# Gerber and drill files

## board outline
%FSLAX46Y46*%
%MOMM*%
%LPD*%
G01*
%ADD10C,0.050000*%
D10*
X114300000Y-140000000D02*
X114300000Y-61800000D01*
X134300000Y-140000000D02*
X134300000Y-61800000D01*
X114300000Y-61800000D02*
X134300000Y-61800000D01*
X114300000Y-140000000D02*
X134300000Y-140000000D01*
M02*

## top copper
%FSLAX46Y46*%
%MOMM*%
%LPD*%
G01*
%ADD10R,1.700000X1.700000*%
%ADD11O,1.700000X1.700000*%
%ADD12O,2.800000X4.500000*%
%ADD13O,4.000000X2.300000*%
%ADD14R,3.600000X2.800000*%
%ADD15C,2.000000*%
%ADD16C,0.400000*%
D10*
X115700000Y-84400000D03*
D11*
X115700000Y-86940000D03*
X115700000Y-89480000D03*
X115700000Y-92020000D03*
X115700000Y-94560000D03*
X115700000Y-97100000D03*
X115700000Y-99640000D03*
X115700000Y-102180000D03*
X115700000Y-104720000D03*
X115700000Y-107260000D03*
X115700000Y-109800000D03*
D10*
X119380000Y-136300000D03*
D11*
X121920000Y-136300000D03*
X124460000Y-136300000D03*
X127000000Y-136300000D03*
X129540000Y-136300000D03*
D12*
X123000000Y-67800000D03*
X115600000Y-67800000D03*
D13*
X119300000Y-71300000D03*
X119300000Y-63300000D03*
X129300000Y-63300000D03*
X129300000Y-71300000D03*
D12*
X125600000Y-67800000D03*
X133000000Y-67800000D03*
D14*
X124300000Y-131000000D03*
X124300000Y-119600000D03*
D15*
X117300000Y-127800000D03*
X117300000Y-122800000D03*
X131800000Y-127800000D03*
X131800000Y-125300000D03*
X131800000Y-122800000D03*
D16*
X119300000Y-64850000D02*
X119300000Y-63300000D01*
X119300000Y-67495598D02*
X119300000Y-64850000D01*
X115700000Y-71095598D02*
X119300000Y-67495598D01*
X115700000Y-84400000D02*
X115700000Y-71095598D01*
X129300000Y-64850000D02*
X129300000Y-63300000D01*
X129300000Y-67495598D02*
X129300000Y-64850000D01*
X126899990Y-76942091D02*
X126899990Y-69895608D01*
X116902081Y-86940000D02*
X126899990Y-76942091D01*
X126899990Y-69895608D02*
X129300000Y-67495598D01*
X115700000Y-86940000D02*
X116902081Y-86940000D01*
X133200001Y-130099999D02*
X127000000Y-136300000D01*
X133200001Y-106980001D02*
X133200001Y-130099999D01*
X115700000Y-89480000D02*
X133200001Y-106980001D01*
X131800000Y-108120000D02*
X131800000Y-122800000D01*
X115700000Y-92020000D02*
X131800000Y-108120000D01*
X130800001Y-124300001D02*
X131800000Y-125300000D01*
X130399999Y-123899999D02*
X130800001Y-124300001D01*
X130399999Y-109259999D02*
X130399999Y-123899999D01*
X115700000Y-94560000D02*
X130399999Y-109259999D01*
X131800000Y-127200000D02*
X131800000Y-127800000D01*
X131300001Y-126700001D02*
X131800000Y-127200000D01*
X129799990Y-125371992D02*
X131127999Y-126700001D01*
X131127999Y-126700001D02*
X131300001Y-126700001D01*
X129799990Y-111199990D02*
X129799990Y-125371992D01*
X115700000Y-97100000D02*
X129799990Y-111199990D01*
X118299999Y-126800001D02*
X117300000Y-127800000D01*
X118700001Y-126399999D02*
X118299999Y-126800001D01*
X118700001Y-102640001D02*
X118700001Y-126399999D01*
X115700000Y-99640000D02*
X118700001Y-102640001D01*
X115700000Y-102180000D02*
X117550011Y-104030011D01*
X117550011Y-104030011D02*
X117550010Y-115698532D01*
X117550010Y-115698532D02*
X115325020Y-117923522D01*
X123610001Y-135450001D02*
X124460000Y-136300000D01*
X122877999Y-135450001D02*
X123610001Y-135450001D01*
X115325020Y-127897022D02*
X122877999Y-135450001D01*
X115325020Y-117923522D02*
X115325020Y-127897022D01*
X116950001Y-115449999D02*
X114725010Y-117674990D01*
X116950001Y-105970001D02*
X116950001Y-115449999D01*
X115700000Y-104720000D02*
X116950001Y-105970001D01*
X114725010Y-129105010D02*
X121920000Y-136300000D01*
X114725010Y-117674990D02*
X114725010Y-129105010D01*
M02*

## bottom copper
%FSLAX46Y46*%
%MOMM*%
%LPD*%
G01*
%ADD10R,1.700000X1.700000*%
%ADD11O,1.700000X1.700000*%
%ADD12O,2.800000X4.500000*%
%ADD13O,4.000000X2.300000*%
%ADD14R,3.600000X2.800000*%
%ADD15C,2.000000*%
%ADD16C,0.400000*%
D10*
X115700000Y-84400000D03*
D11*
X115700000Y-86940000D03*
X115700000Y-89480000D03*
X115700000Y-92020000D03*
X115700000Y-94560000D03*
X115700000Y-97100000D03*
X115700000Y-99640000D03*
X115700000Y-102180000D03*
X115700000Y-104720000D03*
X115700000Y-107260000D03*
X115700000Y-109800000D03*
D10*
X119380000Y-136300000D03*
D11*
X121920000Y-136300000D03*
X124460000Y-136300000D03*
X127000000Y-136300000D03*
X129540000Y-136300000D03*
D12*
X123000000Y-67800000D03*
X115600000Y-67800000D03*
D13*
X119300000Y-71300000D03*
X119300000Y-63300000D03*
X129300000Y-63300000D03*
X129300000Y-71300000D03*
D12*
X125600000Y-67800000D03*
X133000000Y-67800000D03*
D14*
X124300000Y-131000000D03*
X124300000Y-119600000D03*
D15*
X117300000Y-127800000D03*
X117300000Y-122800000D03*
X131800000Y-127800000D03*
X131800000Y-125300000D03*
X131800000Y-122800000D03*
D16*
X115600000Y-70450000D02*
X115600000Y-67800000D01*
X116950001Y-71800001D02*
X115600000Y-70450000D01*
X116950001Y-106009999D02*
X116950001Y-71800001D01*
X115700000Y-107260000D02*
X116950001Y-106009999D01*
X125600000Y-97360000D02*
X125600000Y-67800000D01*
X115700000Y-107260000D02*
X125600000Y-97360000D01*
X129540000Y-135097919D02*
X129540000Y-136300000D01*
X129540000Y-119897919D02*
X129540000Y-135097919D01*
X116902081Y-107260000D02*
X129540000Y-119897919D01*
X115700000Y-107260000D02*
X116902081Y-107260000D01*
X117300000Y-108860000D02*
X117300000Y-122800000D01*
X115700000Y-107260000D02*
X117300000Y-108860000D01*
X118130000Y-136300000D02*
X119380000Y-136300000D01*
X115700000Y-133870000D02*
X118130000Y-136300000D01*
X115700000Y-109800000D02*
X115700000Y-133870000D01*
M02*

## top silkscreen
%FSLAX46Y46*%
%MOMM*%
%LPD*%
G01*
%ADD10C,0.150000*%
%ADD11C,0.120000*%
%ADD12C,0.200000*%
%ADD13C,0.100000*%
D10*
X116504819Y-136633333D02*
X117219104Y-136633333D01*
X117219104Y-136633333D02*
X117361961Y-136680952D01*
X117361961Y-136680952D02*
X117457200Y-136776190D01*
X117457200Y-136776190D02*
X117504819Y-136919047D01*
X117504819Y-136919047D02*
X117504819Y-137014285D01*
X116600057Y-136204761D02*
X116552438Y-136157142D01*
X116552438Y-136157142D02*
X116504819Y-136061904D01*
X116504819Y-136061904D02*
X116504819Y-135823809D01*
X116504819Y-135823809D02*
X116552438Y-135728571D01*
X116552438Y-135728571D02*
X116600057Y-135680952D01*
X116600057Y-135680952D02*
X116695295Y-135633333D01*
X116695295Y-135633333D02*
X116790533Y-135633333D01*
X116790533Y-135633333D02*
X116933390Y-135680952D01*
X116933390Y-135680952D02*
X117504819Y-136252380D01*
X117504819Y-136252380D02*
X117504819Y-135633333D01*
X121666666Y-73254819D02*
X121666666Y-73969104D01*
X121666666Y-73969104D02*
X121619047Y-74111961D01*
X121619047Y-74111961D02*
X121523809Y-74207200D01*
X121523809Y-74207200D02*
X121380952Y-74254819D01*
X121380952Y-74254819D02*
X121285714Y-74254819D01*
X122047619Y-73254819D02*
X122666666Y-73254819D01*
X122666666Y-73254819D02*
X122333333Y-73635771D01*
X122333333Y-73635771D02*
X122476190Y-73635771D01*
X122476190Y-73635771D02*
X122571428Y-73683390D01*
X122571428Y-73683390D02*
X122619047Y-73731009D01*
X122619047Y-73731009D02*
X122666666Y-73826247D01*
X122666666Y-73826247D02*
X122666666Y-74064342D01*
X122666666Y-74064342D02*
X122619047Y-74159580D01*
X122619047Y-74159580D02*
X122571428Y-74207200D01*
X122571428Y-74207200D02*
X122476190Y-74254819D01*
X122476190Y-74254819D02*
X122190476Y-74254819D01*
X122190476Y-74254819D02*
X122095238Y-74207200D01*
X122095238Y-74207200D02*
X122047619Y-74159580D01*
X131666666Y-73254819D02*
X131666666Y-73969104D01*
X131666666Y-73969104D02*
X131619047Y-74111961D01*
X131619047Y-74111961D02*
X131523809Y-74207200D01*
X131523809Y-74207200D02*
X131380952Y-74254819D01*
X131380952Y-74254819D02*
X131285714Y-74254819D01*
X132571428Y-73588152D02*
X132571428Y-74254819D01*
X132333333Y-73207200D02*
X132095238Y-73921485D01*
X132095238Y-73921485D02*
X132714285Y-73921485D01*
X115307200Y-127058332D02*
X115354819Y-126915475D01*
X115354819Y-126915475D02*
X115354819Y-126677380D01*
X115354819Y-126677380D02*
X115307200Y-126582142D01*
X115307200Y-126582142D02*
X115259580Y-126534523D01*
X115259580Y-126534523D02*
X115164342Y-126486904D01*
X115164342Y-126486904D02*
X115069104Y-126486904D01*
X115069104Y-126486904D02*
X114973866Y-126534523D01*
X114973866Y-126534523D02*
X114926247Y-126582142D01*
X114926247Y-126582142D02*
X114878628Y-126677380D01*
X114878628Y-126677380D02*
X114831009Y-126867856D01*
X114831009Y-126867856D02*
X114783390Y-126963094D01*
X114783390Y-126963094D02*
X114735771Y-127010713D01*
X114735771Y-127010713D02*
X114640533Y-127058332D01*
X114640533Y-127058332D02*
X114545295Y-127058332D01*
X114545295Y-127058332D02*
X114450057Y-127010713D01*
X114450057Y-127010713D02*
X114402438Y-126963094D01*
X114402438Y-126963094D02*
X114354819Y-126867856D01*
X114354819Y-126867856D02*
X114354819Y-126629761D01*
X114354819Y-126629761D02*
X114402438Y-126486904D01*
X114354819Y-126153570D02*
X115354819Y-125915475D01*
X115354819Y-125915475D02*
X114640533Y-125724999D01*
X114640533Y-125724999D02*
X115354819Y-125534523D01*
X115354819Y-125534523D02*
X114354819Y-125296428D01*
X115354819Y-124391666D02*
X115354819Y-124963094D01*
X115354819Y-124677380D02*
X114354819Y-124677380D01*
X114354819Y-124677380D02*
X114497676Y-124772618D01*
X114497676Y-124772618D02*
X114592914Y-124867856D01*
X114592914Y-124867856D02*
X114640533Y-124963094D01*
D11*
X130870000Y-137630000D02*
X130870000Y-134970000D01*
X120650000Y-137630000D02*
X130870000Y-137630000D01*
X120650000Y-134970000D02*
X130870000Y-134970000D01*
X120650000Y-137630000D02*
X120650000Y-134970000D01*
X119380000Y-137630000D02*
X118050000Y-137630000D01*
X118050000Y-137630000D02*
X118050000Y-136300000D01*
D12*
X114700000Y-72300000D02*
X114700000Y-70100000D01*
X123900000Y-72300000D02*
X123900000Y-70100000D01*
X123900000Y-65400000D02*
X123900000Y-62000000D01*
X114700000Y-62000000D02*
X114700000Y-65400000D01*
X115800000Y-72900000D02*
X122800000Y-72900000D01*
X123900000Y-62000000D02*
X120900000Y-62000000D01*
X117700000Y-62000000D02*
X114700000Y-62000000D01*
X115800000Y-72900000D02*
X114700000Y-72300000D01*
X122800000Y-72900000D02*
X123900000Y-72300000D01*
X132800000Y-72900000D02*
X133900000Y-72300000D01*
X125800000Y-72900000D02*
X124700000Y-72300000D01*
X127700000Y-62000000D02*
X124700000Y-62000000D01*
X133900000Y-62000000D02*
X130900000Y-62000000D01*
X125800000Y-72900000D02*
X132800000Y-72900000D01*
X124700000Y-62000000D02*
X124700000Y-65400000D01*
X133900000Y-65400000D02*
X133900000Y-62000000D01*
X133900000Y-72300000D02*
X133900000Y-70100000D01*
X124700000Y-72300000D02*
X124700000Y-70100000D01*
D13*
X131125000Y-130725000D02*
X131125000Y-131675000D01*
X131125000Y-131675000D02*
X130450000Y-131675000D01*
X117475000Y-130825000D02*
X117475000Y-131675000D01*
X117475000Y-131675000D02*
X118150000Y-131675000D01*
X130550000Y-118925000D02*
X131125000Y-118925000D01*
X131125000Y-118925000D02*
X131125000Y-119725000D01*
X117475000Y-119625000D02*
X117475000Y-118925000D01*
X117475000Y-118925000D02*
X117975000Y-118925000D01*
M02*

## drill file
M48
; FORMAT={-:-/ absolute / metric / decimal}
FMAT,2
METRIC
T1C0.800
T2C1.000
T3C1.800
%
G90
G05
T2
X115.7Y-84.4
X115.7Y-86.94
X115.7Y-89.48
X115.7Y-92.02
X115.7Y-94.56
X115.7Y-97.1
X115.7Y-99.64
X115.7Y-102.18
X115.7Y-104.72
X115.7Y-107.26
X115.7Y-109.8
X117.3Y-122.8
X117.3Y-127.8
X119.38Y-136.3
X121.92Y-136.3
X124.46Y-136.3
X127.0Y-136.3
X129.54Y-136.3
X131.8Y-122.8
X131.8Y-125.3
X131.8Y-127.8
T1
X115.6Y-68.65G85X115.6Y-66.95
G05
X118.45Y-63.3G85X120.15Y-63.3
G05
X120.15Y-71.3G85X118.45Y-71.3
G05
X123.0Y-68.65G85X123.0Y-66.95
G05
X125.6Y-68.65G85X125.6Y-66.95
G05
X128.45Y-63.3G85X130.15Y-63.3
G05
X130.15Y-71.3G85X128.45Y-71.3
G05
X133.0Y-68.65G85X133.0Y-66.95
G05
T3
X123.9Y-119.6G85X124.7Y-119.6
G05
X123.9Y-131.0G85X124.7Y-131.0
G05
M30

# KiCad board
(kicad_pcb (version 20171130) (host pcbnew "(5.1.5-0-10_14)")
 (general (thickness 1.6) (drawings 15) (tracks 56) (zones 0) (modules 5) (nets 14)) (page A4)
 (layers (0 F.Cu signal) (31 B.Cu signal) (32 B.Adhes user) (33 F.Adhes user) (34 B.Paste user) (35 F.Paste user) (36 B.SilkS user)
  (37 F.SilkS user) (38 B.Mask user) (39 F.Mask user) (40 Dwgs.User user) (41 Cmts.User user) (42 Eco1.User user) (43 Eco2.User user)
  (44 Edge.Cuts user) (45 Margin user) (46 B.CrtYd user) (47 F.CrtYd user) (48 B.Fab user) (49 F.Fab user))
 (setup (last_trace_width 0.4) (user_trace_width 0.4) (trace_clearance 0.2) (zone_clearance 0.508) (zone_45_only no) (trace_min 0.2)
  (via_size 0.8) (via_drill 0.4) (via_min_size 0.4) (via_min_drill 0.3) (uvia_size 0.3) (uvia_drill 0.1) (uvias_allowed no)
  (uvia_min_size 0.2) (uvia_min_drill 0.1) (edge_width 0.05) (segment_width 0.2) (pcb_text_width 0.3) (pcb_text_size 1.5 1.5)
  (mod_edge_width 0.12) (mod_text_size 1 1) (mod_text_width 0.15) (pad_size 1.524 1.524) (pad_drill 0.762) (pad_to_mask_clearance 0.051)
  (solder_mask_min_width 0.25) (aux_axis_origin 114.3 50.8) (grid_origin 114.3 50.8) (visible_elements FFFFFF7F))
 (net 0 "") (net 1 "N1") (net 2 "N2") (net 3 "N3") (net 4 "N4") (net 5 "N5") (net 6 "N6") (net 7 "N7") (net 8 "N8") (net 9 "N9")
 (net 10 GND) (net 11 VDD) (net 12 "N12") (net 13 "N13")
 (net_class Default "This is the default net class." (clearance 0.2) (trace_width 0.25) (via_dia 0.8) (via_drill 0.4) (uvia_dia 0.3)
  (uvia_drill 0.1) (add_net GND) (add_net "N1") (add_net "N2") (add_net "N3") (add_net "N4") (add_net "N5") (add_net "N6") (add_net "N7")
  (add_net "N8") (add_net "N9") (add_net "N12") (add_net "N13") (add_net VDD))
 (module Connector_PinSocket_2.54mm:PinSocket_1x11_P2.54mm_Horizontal (layer B.Cu) (at 115.7 84.4 180)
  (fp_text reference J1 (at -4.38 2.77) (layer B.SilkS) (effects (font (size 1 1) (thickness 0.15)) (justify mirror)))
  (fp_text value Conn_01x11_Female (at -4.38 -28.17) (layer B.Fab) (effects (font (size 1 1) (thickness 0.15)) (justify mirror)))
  (pad 1 thru_hole rect (at 0 0 180) (size 1.7 1.7) (drill 1) (layers *.Cu *.Mask) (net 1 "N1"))
  (pad 2 thru_hole oval (at 0 -2.54 180) (size 1.7 1.7) (drill 1) (layers *.Cu *.Mask) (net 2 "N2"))
  (pad 3 thru_hole oval (at 0 -5.08 180) (size 1.7 1.7) (drill 1) (layers *.Cu *.Mask) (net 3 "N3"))
  (pad 4 thru_hole oval (at 0 -7.62 180) (size 1.7 1.7) (drill 1) (layers *.Cu *.Mask) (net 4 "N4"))
  (pad 5 thru_hole oval (at 0 -10.16 180) (size 1.7 1.7) (drill 1) (layers *.Cu *.Mask) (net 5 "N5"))
  (pad 6 thru_hole oval (at 0 -12.7 180) (size 1.7 1.7) (drill 1) (layers *.Cu *.Mask) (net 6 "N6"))
  (pad 7 thru_hole oval (at 0 -15.24 180) (size 1.7 1.7) (drill 1) (layers *.Cu *.Mask) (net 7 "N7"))
  (pad 8 thru_hole oval (at 0 -17.78 180) (size 1.7 1.7) (drill 1) (layers *.Cu *.Mask) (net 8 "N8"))
  (pad 9 thru_hole oval (at 0 -20.32 180) (size 1.7 1.7) (drill 1) (layers *.Cu *.Mask) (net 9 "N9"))
  (pad 10 thru_hole oval (at 0 -22.86 180) (size 1.7 1.7) (drill 1) (layers *.Cu *.Mask) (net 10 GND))
  (pad 11 thru_hole oval (at 0 -25.4 180) (size 1.7 1.7) (drill 1) (layers *.Cu *.Mask) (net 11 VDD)))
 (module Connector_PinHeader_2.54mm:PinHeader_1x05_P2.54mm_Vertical (layer F.Cu) (at 119.38 136.3 90)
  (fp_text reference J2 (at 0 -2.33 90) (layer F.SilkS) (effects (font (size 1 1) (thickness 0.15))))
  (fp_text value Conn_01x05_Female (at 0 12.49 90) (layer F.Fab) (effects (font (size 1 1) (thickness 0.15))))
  (fp_line (start -1.33 11.49) (end 1.33 11.49) (layer F.SilkS) (width 0.12))
  (fp_line (start -1.33 1.27) (end -1.33 11.49) (layer F.SilkS) (width 0.12))
  (fp_line (start 1.33 1.27) (end 1.33 11.49) (layer F.SilkS) (width 0.12))
  (fp_line (start -1.33 1.27) (end 1.33 1.27) (layer F.SilkS) (width 0.12))
  (fp_line (start -1.33 0) (end -1.33 -1.33) (layer F.SilkS) (width 0.12))
  (fp_line (start -1.33 -1.33) (end 0 -1.33) (layer F.SilkS) (width 0.12))
  (pad 1 thru_hole rect (at 0 0 90) (size 1.7 1.7) (drill 1) (layers *.Cu *.Mask) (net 11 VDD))
  (pad 2 thru_hole oval (at 0 2.54 90) (size 1.7 1.7) (drill 1) (layers *.Cu *.Mask) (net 9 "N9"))
  (pad 3 thru_hole oval (at 0 5.08 90) (size 1.7 1.7) (drill 1) (layers *.Cu *.Mask) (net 8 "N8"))
  (pad 4 thru_hole oval (at 0 7.62 90) (size 1.7 1.7) (drill 1) (layers *.Cu *.Mask) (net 3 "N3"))
  (pad 5 thru_hole oval (at 0 10.16 90) (size 1.7 1.7) (drill 1) (layers *.Cu *.Mask) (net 10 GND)))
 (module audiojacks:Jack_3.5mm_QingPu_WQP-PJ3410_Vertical (layer F.Cu) (at 119.3 67.8 180)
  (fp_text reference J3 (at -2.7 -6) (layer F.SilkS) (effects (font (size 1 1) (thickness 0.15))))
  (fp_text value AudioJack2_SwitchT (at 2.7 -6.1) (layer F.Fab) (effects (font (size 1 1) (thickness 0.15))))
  (fp_line (start 4.6 -4.5) (end 4.6 -2.3) (layer F.SilkS) (width 0.2))
  (fp_line (start -4.6 -4.5) (end -4.6 -2.3) (layer F.SilkS) (width 0.2))
  (fp_line (start -4.6 2.4) (end -4.6 5.8) (layer F.SilkS) (width 0.2))
  (fp_line (start 4.6 5.8) (end 4.6 2.4) (layer F.SilkS) (width 0.2))
  (fp_line (start 3.5 -5.1) (end -3.5 -5.1) (layer F.SilkS) (width 0.2))
  (fp_line (start -4.6 5.8) (end -1.6 5.8) (layer F.SilkS) (width 0.2))
  (fp_line (start 1.6 5.8) (end 4.6 5.8) (layer F.SilkS) (width 0.2))
  (fp_line (start 3.5 -5.1) (end 4.6 -4.5) (layer F.SilkS) (width 0.2))
  (fp_line (start -3.5 -5.1) (end -4.6 -4.5) (layer F.SilkS) (width 0.2))
  (pad TN thru_hole oval (at -3.7 0 180) (size 2.8 4.5) (drill oval 0.8 2.5) (layers *.Cu *.Mask) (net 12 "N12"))
  (pad S thru_hole oval (at 3.7 0 180) (size 2.8 4.5) (drill oval 0.8 2.5) (layers *.Cu *.Mask) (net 10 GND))
  (pad R thru_hole oval (at 0 -3.5 270) (size 2.3 4) (drill oval 0.8 2.5) (layers *.Cu *.Mask))
  (pad T thru_hole oval (at 0 4.5 90) (size 2.3 4) (drill oval 0.8 2.5) (layers *.Cu *.Mask) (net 1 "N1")))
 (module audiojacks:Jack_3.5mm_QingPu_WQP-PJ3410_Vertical (layer F.Cu) (at 129.3 67.8 180)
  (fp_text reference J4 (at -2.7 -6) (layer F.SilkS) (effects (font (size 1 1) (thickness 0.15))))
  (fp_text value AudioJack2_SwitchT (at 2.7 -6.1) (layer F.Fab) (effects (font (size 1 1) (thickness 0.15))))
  (fp_line (start -3.5 -5.1) (end -4.6 -4.5) (layer F.SilkS) (width 0.2))
  (fp_line (start 3.5 -5.1) (end 4.6 -4.5) (layer F.SilkS) (width 0.2))
  (fp_line (start 1.6 5.8) (end 4.6 5.8) (layer F.SilkS) (width 0.2))
  (fp_line (start -4.6 5.8) (end -1.6 5.8) (layer F.SilkS) (width 0.2))
  (fp_line (start 3.5 -5.1) (end -3.5 -5.1) (layer F.SilkS) (width 0.2))
  (fp_line (start 4.6 5.8) (end 4.6 2.4) (layer F.SilkS) (width 0.2))
  (fp_line (start -4.6 2.4) (end -4.6 5.8) (layer F.SilkS) (width 0.2))
  (fp_line (start -4.6 -4.5) (end -4.6 -2.3) (layer F.SilkS) (width 0.2))
  (fp_line (start 4.6 -4.5) (end 4.6 -2.3) (layer F.SilkS) (width 0.2))
  (pad T thru_hole oval (at 0 4.5 90) (size 2.3 4) (drill oval 0.8 2.5) (layers *.Cu *.Mask) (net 2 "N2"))
  (pad R thru_hole oval (at 0 -3.5 270) (size 2.3 4) (drill oval 0.8 2.5) (layers *.Cu *.Mask))
  (pad S thru_hole oval (at 3.7 0 180) (size 2.8 4.5) (drill oval 0.8 2.5) (layers *.Cu *.Mask) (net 10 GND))
  (pad TN thru_hole oval (at -3.7 0 180) (size 2.8 4.5) (drill oval 0.8 2.5) (layers *.Cu *.Mask) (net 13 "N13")))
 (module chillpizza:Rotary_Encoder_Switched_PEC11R (layer F.Cu) (at 124.3 131 90)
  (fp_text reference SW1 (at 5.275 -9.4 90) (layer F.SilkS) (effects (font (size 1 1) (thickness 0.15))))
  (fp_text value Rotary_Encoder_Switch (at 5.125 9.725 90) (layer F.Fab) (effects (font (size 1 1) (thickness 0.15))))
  (fp_line (start 0.275 6.825) (end -0.675 6.825) (layer F.SilkS) (width 0.1))
  (fp_line (start -0.675 6.825) (end -0.675 6.15) (layer F.SilkS) (width 0.1))
  (fp_line (start 0.175 -6.825) (end -0.675 -6.825) (layer F.SilkS) (width 0.1))
  (fp_line (start -0.675 -6.825) (end -0.675 -6.15) (layer F.SilkS) (width 0.1))
  (fp_line (start 12.075 6.25) (end 12.075 6.825) (layer F.SilkS) (width 0.1))
  (fp_line (start 12.075 6.825) (end 11.275 6.825) (layer F.SilkS) (width 0.1))
  (fp_line (start 11.375 -6.825) (end 12.075 -6.825) (layer F.SilkS) (width 0.1))
  (fp_line (start 12.075 -6.825) (end 12.075 -6.325) (layer F.SilkS) (width 0.1))
  (pad 3 thru_hole rect (at 0 0 90) (size 2.8 3.6) (drill oval 1.8 2.6) (layers *.Cu *.Mask))
  (pad 3 thru_hole rect (at 11.4 0 90) (size 2.8 3.6) (drill oval 1.8 2.6) (layers *.Cu *.Mask))
  (pad S1 thru_hole circle (at 3.2 -7 90) (size 2 2) (drill 1) (layers *.Cu *.Mask) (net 7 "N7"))
  (pad S2 thru_hole circle (at 8.2 -7 90) (size 2 2) (drill 1) (layers *.Cu *.Mask) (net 10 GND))
  (pad A thru_hole circle (at 3.2 7.5 90) (size 2 2) (drill 1) (layers *.Cu *.Mask) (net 6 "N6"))
  (pad C thru_hole circle (at 5.7 7.5 90) (size 2 2) (drill 1) (layers *.Cu *.Mask) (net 5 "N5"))
  (pad B thru_hole circle (at 8.2 7.5 90) (size 2 2) (drill 1) (layers *.Cu *.Mask) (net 4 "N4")))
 (gr_line (start 114.3 140) (end 114.3 61.8) (layer Edge.Cuts) (width 0.05))
 (gr_line (start 134.3 140) (end 134.3 61.8) (layer Edge.Cuts) (width 0.05))
 (gr_line (start 114.3 61.8) (end 134.3 61.8) (layer Edge.Cuts) (width 0.05))
 (gr_line (start 114.3 140) (end 134.3 140) (layer Edge.Cuts) (width 0.05))
 (segment (start 119.3 64.85) (end 119.3 63.3) (width 0.4) (layer F.Cu) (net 1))
 (segment (start 119.3 67.495598) (end 119.3 64.85) (width 0.4) (layer F.Cu) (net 1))
 (segment (start 115.7 71.095598) (end 119.3 67.495598) (width 0.4) (layer F.Cu) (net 1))
 (segment (start 115.7 84.4) (end 115.7 71.095598) (width 0.4) (layer F.Cu) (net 1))
 (segment (start 129.3 64.85) (end 129.3 63.3) (width 0.4) (layer F.Cu) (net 2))
 (segment (start 129.3 67.495598) (end 129.3 64.85) (width 0.4) (layer F.Cu) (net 2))
 (segment (start 126.89999 76.942091) (end 126.89999 69.895608) (width 0.4) (layer F.Cu) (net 2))
 (segment (start 116.902081 86.94) (end 126.89999 76.942091) (width 0.4) (layer F.Cu) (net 2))
 (segment (start 126.89999 69.895608) (end 129.3 67.495598) (width 0.4) (layer F.Cu) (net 2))
 (segment (start 115.7 86.94) (end 116.902081 86.94) (width 0.4) (layer F.Cu) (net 2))
 (segment (start 133.200001 130.099999) (end 127 136.3) (width 0.4) (layer F.Cu) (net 3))
 (segment (start 133.200001 106.980001) (end 133.200001 130.099999) (width 0.4) (layer F.Cu) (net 3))
 (segment (start 115.7 89.48) (end 133.200001 106.980001) (width 0.4) (layer F.Cu) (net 3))
 (segment (start 131.8 108.12) (end 131.8 122.8) (width 0.4) (layer F.Cu) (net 4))
 (segment (start 115.7 92.02) (end 131.8 108.12) (width 0.4) (layer F.Cu) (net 4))
 (segment (start 130.800001 124.300001) (end 131.8 125.3) (width 0.4) (layer F.Cu) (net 5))
 (segment (start 130.399999 123.899999) (end 130.800001 124.300001) (width 0.4) (layer F.Cu) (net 5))
 (segment (start 130.399999 109.259999) (end 130.399999 123.899999) (width 0.4) (layer F.Cu) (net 5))
 (segment (start 115.7 94.56) (end 130.399999 109.259999) (width 0.4) (layer F.Cu) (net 5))
 (segment (start 131.8 127.2) (end 131.8 127.8) (width 0.4) (layer F.Cu) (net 6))
 (segment (start 131.300001 126.700001) (end 131.8 127.2) (width 0.4) (layer F.Cu) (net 6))
 (segment (start 129.79999 125.371992) (end 131.127999 126.700001) (width 0.4) (layer F.Cu) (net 6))
 (segment (start 131.127999 126.700001) (end 131.300001 126.700001) (width 0.4) (layer F.Cu) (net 6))
 (segment (start 129.79999 111.19999) (end 129.79999 125.371992) (width 0.4) (layer F.Cu) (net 6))
 (segment (start 115.7 97.1) (end 129.79999 111.19999) (width 0.4) (layer F.Cu) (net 6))
 (segment (start 118.299999 126.800001) (end 117.3 127.8) (width 0.4) (layer F.Cu) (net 7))
 (segment (start 118.700001 126.399999) (end 118.299999 126.800001) (width 0.4) (layer F.Cu) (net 7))
 (segment (start 118.700001 102.640001) (end 118.700001 126.399999) (width 0.4) (layer F.Cu) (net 7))
 (segment (start 115.7 99.64) (end 118.700001 102.640001) (width 0.4) (layer F.Cu) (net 7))
 (segment (start 115.7 102.18) (end 117.550011 104.030011) (width 0.4) (layer F.Cu) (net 8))
 (segment (start 117.550011 104.030011) (end 117.55001 115.698532) (width 0.4) (layer F.Cu) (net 8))
 (segment (start 117.55001 115.698532) (end 115.32502 117.923522) (width 0.4) (layer F.Cu) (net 8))
 (segment (start 123.610001 135.450001) (end 124.46 136.3) (width 0.4) (layer F.Cu) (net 8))
 (segment (start 122.877999 135.450001) (end 123.610001 135.450001) (width 0.4) (layer F.Cu) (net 8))
 (segment (start 115.32502 127.897022) (end 122.877999 135.450001) (width 0.4) (layer F.Cu) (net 8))
 (segment (start 115.32502 117.923522) (end 115.32502 127.897022) (width 0.4) (layer F.Cu) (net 8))
 (segment (start 116.950001 115.449999) (end 114.72501 117.67499) (width 0.4) (layer F.Cu) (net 9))
 (segment (start 116.950001 105.970001) (end 116.950001 115.449999) (width 0.4) (layer F.Cu) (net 9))
 (segment (start 115.7 104.72) (end 116.950001 105.970001) (width 0.4) (layer F.Cu) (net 9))
 (segment (start 114.72501 129.10501) (end 121.92 136.3) (width 0.4) (layer F.Cu) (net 9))
 (segment (start 114.72501 117.67499) (end 114.72501 129.10501) (width 0.4) (layer F.Cu) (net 9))
 (segment (start 115.6 70.45) (end 115.6 67.8) (width 0.4) (layer B.Cu) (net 10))
 (segment (start 116.950001 71.800001) (end 115.6 70.45) (width 0.4) (layer B.Cu) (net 10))
 (segment (start 116.950001 106.009999) (end 116.950001 71.800001) (width 0.4) (layer B.Cu) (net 10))
 (segment (start 115.7 107.26) (end 116.950001 106.009999) (width 0.4) (layer B.Cu) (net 10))
 (segment (start 125.6 97.36) (end 125.6 67.8) (width 0.4) (layer B.Cu) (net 10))
 (segment (start 115.7 107.26) (end 125.6 97.36) (width 0.4) (layer B.Cu) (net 10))
 (segment (start 129.54 135.097919) (end 129.54 136.3) (width 0.4) (layer B.Cu) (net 10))
 (segment (start 129.54 119.897919) (end 129.54 135.097919) (width 0.4) (layer B.Cu) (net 10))
 (segment (start 116.902081 107.26) (end 129.54 119.897919) (width 0.4) (layer B.Cu) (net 10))
 (segment (start 115.7 107.26) (end 116.902081 107.26) (width 0.4) (layer B.Cu) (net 10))
 (segment (start 117.3 108.86) (end 117.3 122.8) (width 0.4) (layer B.Cu) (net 10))
 (segment (start 115.7 107.26) (end 117.3 108.86) (width 0.4) (layer B.Cu) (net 10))
 (segment (start 118.13 136.3) (end 119.38 136.3) (width 0.4) (layer B.Cu) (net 11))
 (segment (start 115.7 133.87) (end 118.13 136.3) (width 0.4) (layer B.Cu) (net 11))
 (segment (start 115.7 109.8) (end 115.7 133.87) (width 0.4) (layer B.Cu) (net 11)))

